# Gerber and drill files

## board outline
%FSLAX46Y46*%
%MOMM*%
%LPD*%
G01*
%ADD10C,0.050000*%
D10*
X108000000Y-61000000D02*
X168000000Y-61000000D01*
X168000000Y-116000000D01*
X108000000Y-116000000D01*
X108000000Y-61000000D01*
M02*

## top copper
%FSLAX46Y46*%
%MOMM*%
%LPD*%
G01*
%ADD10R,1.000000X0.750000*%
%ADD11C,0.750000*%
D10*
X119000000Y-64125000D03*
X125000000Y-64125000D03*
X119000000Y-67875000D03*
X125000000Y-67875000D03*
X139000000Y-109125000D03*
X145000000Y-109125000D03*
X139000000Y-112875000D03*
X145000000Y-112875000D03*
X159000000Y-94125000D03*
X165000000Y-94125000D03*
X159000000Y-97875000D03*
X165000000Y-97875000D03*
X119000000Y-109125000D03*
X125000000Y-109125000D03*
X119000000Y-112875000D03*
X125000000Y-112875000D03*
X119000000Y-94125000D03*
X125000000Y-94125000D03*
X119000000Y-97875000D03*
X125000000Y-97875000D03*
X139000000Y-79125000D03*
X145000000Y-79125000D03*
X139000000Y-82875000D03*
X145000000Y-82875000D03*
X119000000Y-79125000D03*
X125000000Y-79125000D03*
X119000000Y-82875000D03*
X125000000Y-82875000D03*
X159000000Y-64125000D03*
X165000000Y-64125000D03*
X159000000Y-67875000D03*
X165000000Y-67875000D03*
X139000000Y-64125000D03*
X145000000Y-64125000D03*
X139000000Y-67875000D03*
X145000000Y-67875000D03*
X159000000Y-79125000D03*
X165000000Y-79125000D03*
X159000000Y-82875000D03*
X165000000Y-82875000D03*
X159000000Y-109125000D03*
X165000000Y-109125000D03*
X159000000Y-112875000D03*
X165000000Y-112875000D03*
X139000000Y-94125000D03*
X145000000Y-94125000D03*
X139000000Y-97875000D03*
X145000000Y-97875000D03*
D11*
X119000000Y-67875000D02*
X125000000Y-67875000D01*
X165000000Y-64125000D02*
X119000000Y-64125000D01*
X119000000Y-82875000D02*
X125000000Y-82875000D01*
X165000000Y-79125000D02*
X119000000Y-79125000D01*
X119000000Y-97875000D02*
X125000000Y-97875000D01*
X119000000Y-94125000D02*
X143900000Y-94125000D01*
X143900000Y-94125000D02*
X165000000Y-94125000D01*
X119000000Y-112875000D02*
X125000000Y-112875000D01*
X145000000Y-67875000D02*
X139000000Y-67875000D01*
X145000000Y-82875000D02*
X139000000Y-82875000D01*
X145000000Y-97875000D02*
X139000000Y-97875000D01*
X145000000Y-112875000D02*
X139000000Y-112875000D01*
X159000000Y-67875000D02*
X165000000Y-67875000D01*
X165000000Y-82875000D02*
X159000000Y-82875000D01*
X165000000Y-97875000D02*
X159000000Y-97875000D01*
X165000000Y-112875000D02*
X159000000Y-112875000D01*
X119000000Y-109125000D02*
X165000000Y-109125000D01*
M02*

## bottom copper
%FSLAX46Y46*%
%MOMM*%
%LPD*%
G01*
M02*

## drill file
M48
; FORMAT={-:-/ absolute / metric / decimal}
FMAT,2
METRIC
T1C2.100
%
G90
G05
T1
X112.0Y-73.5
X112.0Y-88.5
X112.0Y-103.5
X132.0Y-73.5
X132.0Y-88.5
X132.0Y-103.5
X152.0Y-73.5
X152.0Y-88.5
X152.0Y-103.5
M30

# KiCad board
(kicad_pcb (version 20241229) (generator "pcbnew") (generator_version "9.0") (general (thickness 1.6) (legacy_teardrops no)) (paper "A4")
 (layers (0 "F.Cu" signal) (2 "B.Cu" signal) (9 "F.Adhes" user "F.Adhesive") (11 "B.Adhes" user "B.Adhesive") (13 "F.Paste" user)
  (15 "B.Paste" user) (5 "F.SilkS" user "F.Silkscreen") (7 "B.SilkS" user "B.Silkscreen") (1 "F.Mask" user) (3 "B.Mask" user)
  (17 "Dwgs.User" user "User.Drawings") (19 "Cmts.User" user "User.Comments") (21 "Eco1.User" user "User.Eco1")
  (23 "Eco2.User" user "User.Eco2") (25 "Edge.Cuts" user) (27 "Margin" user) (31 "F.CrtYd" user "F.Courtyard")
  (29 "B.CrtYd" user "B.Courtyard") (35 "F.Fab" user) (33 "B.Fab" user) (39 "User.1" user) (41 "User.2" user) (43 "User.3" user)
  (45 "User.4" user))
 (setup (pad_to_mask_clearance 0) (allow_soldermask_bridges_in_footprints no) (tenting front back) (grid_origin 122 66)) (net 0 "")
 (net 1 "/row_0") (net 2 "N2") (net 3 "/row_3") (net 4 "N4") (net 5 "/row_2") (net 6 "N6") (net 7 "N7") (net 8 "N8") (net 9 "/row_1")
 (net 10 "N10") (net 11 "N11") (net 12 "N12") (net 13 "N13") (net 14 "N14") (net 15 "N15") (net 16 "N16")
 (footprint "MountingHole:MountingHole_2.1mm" (layer "F.Cu") (at 152 103.5)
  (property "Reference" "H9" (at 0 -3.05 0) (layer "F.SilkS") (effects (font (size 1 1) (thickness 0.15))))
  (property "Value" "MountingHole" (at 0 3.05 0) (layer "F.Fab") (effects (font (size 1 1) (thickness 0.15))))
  (pad "" np_thru_hole circle (at 0 0) (size 2.1 2.1) (drill 2.1) (layers "*.Cu" "*.Mask")))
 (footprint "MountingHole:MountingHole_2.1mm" (layer "F.Cu") (at 132 73.5)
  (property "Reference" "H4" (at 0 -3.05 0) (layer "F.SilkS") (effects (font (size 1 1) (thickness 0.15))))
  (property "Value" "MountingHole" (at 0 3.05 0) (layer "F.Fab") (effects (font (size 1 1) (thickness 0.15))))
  (pad "" np_thru_hole circle (at 0 0) (size 2.1 2.1) (drill 2.1) (layers "*.Cu" "*.Mask")))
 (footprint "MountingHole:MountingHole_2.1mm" (layer "F.Cu") (at 112 73.5)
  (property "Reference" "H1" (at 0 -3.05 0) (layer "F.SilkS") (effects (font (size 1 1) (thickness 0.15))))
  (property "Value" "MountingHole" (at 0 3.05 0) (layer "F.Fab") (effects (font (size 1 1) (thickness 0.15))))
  (pad "" np_thru_hole circle (at 0 0) (size 2.1 2.1) (drill 2.1) (layers "*.Cu" "*.Mask")))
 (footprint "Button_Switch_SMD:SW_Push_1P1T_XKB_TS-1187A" (layer "F.Cu") (at 122 66)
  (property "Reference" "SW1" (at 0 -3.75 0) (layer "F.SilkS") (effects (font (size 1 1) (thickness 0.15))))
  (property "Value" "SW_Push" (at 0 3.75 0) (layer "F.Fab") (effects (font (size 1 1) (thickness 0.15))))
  (pad "1" smd rect (at -3 -1.875) (size 1 0.75) (layers "F.Cu" "F.Mask" "F.Paste") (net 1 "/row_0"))
  (pad "1" smd rect (at 3 -1.875) (size 1 0.75) (layers "F.Cu" "F.Mask" "F.Paste") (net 1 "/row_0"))
  (pad "2" smd rect (at -3 1.875) (size 1 0.75) (layers "F.Cu" "F.Mask" "F.Paste") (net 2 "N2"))
  (pad "2" smd rect (at 3 1.875) (size 1 0.75) (layers "F.Cu" "F.Mask" "F.Paste") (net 2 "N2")))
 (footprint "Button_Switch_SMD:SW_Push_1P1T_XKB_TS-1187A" (layer "F.Cu") (at 142 111)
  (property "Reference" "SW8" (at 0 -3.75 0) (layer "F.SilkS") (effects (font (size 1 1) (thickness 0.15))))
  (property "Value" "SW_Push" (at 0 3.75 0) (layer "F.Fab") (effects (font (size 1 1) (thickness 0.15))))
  (pad "1" smd rect (at -3 -1.875) (size 1 0.75) (layers "F.Cu" "F.Mask" "F.Paste") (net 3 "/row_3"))
  (pad "1" smd rect (at 3 -1.875) (size 1 0.75) (layers "F.Cu" "F.Mask" "F.Paste") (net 3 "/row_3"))
  (pad "2" smd rect (at -3 1.875) (size 1 0.75) (layers "F.Cu" "F.Mask" "F.Paste") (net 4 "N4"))
  (pad "2" smd rect (at 3 1.875) (size 1 0.75) (layers "F.Cu" "F.Mask" "F.Paste") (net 4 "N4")))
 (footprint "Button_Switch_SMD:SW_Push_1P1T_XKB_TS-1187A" (layer "F.Cu") (at 162 96)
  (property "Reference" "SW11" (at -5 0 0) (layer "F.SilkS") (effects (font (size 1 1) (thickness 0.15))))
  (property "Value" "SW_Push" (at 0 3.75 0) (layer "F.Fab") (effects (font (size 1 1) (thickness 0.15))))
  (pad "1" smd rect (at -3 -1.875) (size 1 0.75) (layers "F.Cu" "F.Mask" "F.Paste") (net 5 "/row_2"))
  (pad "1" smd rect (at 3 -1.875) (size 1 0.75) (layers "F.Cu" "F.Mask" "F.Paste") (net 5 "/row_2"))
  (pad "2" smd rect (at -3 1.875) (size 1 0.75) (layers "F.Cu" "F.Mask" "F.Paste") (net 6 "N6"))
  (pad "2" smd rect (at 3 1.875) (size 1 0.75) (layers "F.Cu" "F.Mask" "F.Paste") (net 6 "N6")))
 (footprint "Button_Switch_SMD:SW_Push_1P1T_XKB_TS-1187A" (layer "F.Cu") (at 122 111)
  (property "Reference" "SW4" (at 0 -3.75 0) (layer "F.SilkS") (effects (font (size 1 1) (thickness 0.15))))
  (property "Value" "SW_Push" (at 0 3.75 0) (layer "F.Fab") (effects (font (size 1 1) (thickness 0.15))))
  (pad "1" smd rect (at -3 -1.875) (size 1 0.75) (layers "F.Cu" "F.Mask" "F.Paste") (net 3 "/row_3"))
  (pad "1" smd rect (at 3 -1.875) (size 1 0.75) (layers "F.Cu" "F.Mask" "F.Paste") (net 3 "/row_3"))
  (pad "2" smd rect (at -3 1.875) (size 1 0.75) (layers "F.Cu" "F.Mask" "F.Paste") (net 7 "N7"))
  (pad "2" smd rect (at 3 1.875) (size 1 0.75) (layers "F.Cu" "F.Mask" "F.Paste") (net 7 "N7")))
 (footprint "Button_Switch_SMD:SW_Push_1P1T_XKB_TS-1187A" (layer "F.Cu") (at 122 96)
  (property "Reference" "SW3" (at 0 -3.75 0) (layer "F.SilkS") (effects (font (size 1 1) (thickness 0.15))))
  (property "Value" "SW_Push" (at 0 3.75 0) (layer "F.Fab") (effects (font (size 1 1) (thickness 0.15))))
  (pad "1" smd rect (at -3 -1.875) (size 1 0.75) (layers "F.Cu" "F.Mask" "F.Paste") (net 5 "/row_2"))
  (pad "1" smd rect (at 3 -1.875) (size 1 0.75) (layers "F.Cu" "F.Mask" "F.Paste") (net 5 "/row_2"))
  (pad "2" smd rect (at -3 1.875) (size 1 0.75) (layers "F.Cu" "F.Mask" "F.Paste") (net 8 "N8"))
  (pad "2" smd rect (at 3 1.875) (size 1 0.75) (layers "F.Cu" "F.Mask" "F.Paste") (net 8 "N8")))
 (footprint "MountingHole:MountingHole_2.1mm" (layer "F.Cu") (at 132 88.5)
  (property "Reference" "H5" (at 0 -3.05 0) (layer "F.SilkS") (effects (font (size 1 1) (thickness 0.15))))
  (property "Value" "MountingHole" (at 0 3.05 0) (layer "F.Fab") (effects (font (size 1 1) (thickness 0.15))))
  (pad "" np_thru_hole circle (at 0 0) (size 2.1 2.1) (drill 2.1) (layers "*.Cu" "*.Mask")))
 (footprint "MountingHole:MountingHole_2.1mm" (layer "F.Cu") (at 112 88.5)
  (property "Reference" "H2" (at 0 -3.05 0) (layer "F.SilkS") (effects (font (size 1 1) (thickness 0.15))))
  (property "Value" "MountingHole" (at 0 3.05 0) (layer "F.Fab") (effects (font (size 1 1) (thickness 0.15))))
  (pad "" np_thru_hole circle (at 0 0) (size 2.1 2.1) (drill 2.1) (layers "*.Cu" "*.Mask")))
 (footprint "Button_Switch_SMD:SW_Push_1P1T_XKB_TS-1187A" (layer "F.Cu") (at 142 81)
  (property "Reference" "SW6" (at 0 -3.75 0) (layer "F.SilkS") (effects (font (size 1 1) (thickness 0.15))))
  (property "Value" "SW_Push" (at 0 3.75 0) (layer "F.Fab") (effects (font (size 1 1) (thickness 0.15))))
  (pad "1" smd rect (at -3 -1.875) (size 1 0.75) (layers "F.Cu" "F.Mask" "F.Paste") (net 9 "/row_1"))
  (pad "1" smd rect (at 3 -1.875) (size 1 0.75) (layers "F.Cu" "F.Mask" "F.Paste") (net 9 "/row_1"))
  (pad "2" smd rect (at -3 1.875) (size 1 0.75) (layers "F.Cu" "F.Mask" "F.Paste") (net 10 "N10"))
  (pad "2" smd rect (at 3 1.875) (size 1 0.75) (layers "F.Cu" "F.Mask" "F.Paste") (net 10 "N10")))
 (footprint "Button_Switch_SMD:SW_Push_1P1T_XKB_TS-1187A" (layer "F.Cu") (at 122 81)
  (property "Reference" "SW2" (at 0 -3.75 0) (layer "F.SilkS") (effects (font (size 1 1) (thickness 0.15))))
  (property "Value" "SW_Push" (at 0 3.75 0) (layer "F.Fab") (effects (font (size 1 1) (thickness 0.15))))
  (pad "1" smd rect (at -3 -1.875) (size 1 0.75) (layers "F.Cu" "F.Mask" "F.Paste") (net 9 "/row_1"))
  (pad "1" smd rect (at 3 -1.875) (size 1 0.75) (layers "F.Cu" "F.Mask" "F.Paste") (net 9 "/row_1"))
  (pad "2" smd rect (at -3 1.875) (size 1 0.75) (layers "F.Cu" "F.Mask" "F.Paste") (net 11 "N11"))
  (pad "2" smd rect (at 3 1.875) (size 1 0.75) (layers "F.Cu" "F.Mask" "F.Paste") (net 11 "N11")))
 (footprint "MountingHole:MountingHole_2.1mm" (layer "F.Cu") (at 112 103.5)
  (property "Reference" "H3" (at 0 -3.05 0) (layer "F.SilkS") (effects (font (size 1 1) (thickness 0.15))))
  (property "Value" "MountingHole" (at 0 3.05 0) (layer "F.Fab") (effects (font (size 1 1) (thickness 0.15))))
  (pad "" np_thru_hole circle (at 0 0) (size 2.1 2.1) (drill 2.1) (layers "*.Cu" "*.Mask")))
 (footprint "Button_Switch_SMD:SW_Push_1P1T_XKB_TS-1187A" (layer "F.Cu") (at 162 66)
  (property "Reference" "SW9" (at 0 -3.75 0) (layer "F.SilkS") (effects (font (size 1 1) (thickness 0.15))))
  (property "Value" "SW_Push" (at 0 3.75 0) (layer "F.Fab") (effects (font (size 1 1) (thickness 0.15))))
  (pad "1" smd rect (at -3 -1.875) (size 1 0.75) (layers "F.Cu" "F.Mask" "F.Paste") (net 1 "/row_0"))
  (pad "1" smd rect (at 3 -1.875) (size 1 0.75) (layers "F.Cu" "F.Mask" "F.Paste") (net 1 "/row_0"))
  (pad "2" smd rect (at -3 1.875) (size 1 0.75) (layers "F.Cu" "F.Mask" "F.Paste") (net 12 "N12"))
  (pad "2" smd rect (at 3 1.875) (size 1 0.75) (layers "F.Cu" "F.Mask" "F.Paste") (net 12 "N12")))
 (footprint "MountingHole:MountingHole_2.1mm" (layer "F.Cu") (at 152 88.5)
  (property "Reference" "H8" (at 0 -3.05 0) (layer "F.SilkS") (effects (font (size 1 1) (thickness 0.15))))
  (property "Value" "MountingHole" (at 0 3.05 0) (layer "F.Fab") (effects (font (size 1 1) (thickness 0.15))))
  (pad "" np_thru_hole circle (at 0 0) (size 2.1 2.1) (drill 2.1) (layers "*.Cu" "*.Mask")))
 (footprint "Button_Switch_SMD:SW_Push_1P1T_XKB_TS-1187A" (layer "F.Cu") (at 142 66)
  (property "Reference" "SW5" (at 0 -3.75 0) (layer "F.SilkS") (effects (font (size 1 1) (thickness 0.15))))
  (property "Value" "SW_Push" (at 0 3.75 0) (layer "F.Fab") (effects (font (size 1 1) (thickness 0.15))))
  (pad "1" smd rect (at -3 -1.875) (size 1 0.75) (layers "F.Cu" "F.Mask" "F.Paste") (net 1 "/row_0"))
  (pad "1" smd rect (at 3 -1.875) (size 1 0.75) (layers "F.Cu" "F.Mask" "F.Paste") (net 1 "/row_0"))
  (pad "2" smd rect (at -3 1.875) (size 1 0.75) (layers "F.Cu" "F.Mask" "F.Paste") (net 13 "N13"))
  (pad "2" smd rect (at 3 1.875) (size 1 0.75) (layers "F.Cu" "F.Mask" "F.Paste") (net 13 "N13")))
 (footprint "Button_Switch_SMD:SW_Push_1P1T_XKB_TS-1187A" (layer "F.Cu") (at 162 81)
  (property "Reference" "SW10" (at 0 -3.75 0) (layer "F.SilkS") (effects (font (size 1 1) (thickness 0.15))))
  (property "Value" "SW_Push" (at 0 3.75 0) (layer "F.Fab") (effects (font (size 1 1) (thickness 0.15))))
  (pad "1" smd rect (at -3 -1.875) (size 1 0.75) (layers "F.Cu" "F.Mask" "F.Paste") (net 9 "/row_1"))
  (pad "1" smd rect (at 3 -1.875) (size 1 0.75) (layers "F.Cu" "F.Mask" "F.Paste") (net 9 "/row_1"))
  (pad "2" smd rect (at -3 1.875) (size 1 0.75) (layers "F.Cu" "F.Mask" "F.Paste") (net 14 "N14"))
  (pad "2" smd rect (at 3 1.875) (size 1 0.75) (layers "F.Cu" "F.Mask" "F.Paste") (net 14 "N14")))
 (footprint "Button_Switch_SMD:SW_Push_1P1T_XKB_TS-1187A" (layer "F.Cu") (at 162 111)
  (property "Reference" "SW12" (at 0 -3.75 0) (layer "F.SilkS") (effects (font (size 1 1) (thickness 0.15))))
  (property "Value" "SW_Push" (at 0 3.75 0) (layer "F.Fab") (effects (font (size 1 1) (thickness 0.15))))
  (pad "1" smd rect (at -3 -1.875) (size 1 0.75) (layers "F.Cu" "F.Mask" "F.Paste") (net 3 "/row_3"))
  (pad "1" smd rect (at 3 -1.875) (size 1 0.75) (layers "F.Cu" "F.Mask" "F.Paste") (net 3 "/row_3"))
  (pad "2" smd rect (at -3 1.875) (size 1 0.75) (layers "F.Cu" "F.Mask" "F.Paste") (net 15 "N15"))
  (pad "2" smd rect (at 3 1.875) (size 1 0.75) (layers "F.Cu" "F.Mask" "F.Paste") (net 15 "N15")))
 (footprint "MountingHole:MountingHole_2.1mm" (layer "F.Cu") (at 152 73.5)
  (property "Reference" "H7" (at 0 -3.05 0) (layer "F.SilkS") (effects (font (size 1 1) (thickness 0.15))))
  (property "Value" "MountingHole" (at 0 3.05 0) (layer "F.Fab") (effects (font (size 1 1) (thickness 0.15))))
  (pad "" np_thru_hole circle (at 0 0) (size 2.1 2.1) (drill 2.1) (layers "*.Cu" "*.Mask")))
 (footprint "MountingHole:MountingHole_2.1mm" (layer "F.Cu") (at 132 103.5)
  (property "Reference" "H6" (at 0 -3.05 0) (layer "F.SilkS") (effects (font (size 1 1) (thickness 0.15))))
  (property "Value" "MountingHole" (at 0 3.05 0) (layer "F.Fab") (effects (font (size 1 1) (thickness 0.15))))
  (pad "" np_thru_hole circle (at 0 0) (size 2.1 2.1) (drill 2.1) (layers "*.Cu" "*.Mask")))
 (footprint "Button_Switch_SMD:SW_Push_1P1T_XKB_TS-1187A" (layer "F.Cu") (at 142 96)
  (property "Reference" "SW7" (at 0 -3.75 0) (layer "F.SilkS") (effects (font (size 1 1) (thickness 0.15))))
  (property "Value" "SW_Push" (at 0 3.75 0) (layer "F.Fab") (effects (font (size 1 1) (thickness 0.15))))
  (pad "1" smd rect (at -3 -1.875) (size 1 0.75) (layers "F.Cu" "F.Mask" "F.Paste") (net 5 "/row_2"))
  (pad "1" smd rect (at 3 -1.875) (size 1 0.75) (layers "F.Cu" "F.Mask" "F.Paste") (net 5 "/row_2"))
  (pad "2" smd rect (at -3 1.875) (size 1 0.75) (layers "F.Cu" "F.Mask" "F.Paste") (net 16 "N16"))
  (pad "2" smd rect (at 3 1.875) (size 1 0.75) (layers "F.Cu" "F.Mask" "F.Paste") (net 16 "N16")))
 (gr_rect (start 108 61) (end 168 116) (stroke (width 0.05) (type solid)) (fill no) (layer "Edge.Cuts"))
 (segment (start 119 67.875) (end 125 67.875) (width 0.75) (layer "F.Cu") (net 2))
 (segment (start 165 64.125) (end 119 64.125) (width 0.75) (layer "F.Cu") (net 1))
 (segment (start 119 82.875) (end 125 82.875) (width 0.75) (layer "F.Cu") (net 11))
 (segment (start 165 79.125) (end 119 79.125) (width 0.75) (layer "F.Cu") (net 9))
 (segment (start 119 97.875) (end 125 97.875) (width 0.75) (layer "F.Cu") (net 8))
 (segment (start 119 94.125) (end 143.9 94.125) (width 0.75) (layer "F.Cu") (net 5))
 (segment (start 143.9 94.125) (end 165 94.125) (width 0.75) (layer "F.Cu") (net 5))
 (segment (start 119 112.875) (end 125 112.875) (width 0.75) (layer "F.Cu") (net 7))
 (segment (start 145 67.875) (end 139 67.875) (width 0.75) (layer "F.Cu") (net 13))
 (segment (start 145 82.875) (end 139 82.875) (width 0.75) (layer "F.Cu") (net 10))
 (segment (start 145 97.875) (end 139 97.875) (width 0.75) (layer "F.Cu") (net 16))
 (segment (start 145 112.875) (end 139 112.875) (width 0.75) (layer "F.Cu") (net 4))
 (segment (start 159 67.875) (end 165 67.875) (width 0.75) (layer "F.Cu") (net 12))
 (segment (start 165 82.875) (end 159 82.875) (width 0.75) (layer "F.Cu") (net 14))
 (segment (start 165 97.875) (end 159 97.875) (width 0.75) (layer "F.Cu") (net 6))
 (segment (start 165 112.875) (end 159 112.875) (width 0.75) (layer "F.Cu") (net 15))
 (segment (start 119 109.125) (end 165 109.125) (width 0.75) (layer "F.Cu") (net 3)))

